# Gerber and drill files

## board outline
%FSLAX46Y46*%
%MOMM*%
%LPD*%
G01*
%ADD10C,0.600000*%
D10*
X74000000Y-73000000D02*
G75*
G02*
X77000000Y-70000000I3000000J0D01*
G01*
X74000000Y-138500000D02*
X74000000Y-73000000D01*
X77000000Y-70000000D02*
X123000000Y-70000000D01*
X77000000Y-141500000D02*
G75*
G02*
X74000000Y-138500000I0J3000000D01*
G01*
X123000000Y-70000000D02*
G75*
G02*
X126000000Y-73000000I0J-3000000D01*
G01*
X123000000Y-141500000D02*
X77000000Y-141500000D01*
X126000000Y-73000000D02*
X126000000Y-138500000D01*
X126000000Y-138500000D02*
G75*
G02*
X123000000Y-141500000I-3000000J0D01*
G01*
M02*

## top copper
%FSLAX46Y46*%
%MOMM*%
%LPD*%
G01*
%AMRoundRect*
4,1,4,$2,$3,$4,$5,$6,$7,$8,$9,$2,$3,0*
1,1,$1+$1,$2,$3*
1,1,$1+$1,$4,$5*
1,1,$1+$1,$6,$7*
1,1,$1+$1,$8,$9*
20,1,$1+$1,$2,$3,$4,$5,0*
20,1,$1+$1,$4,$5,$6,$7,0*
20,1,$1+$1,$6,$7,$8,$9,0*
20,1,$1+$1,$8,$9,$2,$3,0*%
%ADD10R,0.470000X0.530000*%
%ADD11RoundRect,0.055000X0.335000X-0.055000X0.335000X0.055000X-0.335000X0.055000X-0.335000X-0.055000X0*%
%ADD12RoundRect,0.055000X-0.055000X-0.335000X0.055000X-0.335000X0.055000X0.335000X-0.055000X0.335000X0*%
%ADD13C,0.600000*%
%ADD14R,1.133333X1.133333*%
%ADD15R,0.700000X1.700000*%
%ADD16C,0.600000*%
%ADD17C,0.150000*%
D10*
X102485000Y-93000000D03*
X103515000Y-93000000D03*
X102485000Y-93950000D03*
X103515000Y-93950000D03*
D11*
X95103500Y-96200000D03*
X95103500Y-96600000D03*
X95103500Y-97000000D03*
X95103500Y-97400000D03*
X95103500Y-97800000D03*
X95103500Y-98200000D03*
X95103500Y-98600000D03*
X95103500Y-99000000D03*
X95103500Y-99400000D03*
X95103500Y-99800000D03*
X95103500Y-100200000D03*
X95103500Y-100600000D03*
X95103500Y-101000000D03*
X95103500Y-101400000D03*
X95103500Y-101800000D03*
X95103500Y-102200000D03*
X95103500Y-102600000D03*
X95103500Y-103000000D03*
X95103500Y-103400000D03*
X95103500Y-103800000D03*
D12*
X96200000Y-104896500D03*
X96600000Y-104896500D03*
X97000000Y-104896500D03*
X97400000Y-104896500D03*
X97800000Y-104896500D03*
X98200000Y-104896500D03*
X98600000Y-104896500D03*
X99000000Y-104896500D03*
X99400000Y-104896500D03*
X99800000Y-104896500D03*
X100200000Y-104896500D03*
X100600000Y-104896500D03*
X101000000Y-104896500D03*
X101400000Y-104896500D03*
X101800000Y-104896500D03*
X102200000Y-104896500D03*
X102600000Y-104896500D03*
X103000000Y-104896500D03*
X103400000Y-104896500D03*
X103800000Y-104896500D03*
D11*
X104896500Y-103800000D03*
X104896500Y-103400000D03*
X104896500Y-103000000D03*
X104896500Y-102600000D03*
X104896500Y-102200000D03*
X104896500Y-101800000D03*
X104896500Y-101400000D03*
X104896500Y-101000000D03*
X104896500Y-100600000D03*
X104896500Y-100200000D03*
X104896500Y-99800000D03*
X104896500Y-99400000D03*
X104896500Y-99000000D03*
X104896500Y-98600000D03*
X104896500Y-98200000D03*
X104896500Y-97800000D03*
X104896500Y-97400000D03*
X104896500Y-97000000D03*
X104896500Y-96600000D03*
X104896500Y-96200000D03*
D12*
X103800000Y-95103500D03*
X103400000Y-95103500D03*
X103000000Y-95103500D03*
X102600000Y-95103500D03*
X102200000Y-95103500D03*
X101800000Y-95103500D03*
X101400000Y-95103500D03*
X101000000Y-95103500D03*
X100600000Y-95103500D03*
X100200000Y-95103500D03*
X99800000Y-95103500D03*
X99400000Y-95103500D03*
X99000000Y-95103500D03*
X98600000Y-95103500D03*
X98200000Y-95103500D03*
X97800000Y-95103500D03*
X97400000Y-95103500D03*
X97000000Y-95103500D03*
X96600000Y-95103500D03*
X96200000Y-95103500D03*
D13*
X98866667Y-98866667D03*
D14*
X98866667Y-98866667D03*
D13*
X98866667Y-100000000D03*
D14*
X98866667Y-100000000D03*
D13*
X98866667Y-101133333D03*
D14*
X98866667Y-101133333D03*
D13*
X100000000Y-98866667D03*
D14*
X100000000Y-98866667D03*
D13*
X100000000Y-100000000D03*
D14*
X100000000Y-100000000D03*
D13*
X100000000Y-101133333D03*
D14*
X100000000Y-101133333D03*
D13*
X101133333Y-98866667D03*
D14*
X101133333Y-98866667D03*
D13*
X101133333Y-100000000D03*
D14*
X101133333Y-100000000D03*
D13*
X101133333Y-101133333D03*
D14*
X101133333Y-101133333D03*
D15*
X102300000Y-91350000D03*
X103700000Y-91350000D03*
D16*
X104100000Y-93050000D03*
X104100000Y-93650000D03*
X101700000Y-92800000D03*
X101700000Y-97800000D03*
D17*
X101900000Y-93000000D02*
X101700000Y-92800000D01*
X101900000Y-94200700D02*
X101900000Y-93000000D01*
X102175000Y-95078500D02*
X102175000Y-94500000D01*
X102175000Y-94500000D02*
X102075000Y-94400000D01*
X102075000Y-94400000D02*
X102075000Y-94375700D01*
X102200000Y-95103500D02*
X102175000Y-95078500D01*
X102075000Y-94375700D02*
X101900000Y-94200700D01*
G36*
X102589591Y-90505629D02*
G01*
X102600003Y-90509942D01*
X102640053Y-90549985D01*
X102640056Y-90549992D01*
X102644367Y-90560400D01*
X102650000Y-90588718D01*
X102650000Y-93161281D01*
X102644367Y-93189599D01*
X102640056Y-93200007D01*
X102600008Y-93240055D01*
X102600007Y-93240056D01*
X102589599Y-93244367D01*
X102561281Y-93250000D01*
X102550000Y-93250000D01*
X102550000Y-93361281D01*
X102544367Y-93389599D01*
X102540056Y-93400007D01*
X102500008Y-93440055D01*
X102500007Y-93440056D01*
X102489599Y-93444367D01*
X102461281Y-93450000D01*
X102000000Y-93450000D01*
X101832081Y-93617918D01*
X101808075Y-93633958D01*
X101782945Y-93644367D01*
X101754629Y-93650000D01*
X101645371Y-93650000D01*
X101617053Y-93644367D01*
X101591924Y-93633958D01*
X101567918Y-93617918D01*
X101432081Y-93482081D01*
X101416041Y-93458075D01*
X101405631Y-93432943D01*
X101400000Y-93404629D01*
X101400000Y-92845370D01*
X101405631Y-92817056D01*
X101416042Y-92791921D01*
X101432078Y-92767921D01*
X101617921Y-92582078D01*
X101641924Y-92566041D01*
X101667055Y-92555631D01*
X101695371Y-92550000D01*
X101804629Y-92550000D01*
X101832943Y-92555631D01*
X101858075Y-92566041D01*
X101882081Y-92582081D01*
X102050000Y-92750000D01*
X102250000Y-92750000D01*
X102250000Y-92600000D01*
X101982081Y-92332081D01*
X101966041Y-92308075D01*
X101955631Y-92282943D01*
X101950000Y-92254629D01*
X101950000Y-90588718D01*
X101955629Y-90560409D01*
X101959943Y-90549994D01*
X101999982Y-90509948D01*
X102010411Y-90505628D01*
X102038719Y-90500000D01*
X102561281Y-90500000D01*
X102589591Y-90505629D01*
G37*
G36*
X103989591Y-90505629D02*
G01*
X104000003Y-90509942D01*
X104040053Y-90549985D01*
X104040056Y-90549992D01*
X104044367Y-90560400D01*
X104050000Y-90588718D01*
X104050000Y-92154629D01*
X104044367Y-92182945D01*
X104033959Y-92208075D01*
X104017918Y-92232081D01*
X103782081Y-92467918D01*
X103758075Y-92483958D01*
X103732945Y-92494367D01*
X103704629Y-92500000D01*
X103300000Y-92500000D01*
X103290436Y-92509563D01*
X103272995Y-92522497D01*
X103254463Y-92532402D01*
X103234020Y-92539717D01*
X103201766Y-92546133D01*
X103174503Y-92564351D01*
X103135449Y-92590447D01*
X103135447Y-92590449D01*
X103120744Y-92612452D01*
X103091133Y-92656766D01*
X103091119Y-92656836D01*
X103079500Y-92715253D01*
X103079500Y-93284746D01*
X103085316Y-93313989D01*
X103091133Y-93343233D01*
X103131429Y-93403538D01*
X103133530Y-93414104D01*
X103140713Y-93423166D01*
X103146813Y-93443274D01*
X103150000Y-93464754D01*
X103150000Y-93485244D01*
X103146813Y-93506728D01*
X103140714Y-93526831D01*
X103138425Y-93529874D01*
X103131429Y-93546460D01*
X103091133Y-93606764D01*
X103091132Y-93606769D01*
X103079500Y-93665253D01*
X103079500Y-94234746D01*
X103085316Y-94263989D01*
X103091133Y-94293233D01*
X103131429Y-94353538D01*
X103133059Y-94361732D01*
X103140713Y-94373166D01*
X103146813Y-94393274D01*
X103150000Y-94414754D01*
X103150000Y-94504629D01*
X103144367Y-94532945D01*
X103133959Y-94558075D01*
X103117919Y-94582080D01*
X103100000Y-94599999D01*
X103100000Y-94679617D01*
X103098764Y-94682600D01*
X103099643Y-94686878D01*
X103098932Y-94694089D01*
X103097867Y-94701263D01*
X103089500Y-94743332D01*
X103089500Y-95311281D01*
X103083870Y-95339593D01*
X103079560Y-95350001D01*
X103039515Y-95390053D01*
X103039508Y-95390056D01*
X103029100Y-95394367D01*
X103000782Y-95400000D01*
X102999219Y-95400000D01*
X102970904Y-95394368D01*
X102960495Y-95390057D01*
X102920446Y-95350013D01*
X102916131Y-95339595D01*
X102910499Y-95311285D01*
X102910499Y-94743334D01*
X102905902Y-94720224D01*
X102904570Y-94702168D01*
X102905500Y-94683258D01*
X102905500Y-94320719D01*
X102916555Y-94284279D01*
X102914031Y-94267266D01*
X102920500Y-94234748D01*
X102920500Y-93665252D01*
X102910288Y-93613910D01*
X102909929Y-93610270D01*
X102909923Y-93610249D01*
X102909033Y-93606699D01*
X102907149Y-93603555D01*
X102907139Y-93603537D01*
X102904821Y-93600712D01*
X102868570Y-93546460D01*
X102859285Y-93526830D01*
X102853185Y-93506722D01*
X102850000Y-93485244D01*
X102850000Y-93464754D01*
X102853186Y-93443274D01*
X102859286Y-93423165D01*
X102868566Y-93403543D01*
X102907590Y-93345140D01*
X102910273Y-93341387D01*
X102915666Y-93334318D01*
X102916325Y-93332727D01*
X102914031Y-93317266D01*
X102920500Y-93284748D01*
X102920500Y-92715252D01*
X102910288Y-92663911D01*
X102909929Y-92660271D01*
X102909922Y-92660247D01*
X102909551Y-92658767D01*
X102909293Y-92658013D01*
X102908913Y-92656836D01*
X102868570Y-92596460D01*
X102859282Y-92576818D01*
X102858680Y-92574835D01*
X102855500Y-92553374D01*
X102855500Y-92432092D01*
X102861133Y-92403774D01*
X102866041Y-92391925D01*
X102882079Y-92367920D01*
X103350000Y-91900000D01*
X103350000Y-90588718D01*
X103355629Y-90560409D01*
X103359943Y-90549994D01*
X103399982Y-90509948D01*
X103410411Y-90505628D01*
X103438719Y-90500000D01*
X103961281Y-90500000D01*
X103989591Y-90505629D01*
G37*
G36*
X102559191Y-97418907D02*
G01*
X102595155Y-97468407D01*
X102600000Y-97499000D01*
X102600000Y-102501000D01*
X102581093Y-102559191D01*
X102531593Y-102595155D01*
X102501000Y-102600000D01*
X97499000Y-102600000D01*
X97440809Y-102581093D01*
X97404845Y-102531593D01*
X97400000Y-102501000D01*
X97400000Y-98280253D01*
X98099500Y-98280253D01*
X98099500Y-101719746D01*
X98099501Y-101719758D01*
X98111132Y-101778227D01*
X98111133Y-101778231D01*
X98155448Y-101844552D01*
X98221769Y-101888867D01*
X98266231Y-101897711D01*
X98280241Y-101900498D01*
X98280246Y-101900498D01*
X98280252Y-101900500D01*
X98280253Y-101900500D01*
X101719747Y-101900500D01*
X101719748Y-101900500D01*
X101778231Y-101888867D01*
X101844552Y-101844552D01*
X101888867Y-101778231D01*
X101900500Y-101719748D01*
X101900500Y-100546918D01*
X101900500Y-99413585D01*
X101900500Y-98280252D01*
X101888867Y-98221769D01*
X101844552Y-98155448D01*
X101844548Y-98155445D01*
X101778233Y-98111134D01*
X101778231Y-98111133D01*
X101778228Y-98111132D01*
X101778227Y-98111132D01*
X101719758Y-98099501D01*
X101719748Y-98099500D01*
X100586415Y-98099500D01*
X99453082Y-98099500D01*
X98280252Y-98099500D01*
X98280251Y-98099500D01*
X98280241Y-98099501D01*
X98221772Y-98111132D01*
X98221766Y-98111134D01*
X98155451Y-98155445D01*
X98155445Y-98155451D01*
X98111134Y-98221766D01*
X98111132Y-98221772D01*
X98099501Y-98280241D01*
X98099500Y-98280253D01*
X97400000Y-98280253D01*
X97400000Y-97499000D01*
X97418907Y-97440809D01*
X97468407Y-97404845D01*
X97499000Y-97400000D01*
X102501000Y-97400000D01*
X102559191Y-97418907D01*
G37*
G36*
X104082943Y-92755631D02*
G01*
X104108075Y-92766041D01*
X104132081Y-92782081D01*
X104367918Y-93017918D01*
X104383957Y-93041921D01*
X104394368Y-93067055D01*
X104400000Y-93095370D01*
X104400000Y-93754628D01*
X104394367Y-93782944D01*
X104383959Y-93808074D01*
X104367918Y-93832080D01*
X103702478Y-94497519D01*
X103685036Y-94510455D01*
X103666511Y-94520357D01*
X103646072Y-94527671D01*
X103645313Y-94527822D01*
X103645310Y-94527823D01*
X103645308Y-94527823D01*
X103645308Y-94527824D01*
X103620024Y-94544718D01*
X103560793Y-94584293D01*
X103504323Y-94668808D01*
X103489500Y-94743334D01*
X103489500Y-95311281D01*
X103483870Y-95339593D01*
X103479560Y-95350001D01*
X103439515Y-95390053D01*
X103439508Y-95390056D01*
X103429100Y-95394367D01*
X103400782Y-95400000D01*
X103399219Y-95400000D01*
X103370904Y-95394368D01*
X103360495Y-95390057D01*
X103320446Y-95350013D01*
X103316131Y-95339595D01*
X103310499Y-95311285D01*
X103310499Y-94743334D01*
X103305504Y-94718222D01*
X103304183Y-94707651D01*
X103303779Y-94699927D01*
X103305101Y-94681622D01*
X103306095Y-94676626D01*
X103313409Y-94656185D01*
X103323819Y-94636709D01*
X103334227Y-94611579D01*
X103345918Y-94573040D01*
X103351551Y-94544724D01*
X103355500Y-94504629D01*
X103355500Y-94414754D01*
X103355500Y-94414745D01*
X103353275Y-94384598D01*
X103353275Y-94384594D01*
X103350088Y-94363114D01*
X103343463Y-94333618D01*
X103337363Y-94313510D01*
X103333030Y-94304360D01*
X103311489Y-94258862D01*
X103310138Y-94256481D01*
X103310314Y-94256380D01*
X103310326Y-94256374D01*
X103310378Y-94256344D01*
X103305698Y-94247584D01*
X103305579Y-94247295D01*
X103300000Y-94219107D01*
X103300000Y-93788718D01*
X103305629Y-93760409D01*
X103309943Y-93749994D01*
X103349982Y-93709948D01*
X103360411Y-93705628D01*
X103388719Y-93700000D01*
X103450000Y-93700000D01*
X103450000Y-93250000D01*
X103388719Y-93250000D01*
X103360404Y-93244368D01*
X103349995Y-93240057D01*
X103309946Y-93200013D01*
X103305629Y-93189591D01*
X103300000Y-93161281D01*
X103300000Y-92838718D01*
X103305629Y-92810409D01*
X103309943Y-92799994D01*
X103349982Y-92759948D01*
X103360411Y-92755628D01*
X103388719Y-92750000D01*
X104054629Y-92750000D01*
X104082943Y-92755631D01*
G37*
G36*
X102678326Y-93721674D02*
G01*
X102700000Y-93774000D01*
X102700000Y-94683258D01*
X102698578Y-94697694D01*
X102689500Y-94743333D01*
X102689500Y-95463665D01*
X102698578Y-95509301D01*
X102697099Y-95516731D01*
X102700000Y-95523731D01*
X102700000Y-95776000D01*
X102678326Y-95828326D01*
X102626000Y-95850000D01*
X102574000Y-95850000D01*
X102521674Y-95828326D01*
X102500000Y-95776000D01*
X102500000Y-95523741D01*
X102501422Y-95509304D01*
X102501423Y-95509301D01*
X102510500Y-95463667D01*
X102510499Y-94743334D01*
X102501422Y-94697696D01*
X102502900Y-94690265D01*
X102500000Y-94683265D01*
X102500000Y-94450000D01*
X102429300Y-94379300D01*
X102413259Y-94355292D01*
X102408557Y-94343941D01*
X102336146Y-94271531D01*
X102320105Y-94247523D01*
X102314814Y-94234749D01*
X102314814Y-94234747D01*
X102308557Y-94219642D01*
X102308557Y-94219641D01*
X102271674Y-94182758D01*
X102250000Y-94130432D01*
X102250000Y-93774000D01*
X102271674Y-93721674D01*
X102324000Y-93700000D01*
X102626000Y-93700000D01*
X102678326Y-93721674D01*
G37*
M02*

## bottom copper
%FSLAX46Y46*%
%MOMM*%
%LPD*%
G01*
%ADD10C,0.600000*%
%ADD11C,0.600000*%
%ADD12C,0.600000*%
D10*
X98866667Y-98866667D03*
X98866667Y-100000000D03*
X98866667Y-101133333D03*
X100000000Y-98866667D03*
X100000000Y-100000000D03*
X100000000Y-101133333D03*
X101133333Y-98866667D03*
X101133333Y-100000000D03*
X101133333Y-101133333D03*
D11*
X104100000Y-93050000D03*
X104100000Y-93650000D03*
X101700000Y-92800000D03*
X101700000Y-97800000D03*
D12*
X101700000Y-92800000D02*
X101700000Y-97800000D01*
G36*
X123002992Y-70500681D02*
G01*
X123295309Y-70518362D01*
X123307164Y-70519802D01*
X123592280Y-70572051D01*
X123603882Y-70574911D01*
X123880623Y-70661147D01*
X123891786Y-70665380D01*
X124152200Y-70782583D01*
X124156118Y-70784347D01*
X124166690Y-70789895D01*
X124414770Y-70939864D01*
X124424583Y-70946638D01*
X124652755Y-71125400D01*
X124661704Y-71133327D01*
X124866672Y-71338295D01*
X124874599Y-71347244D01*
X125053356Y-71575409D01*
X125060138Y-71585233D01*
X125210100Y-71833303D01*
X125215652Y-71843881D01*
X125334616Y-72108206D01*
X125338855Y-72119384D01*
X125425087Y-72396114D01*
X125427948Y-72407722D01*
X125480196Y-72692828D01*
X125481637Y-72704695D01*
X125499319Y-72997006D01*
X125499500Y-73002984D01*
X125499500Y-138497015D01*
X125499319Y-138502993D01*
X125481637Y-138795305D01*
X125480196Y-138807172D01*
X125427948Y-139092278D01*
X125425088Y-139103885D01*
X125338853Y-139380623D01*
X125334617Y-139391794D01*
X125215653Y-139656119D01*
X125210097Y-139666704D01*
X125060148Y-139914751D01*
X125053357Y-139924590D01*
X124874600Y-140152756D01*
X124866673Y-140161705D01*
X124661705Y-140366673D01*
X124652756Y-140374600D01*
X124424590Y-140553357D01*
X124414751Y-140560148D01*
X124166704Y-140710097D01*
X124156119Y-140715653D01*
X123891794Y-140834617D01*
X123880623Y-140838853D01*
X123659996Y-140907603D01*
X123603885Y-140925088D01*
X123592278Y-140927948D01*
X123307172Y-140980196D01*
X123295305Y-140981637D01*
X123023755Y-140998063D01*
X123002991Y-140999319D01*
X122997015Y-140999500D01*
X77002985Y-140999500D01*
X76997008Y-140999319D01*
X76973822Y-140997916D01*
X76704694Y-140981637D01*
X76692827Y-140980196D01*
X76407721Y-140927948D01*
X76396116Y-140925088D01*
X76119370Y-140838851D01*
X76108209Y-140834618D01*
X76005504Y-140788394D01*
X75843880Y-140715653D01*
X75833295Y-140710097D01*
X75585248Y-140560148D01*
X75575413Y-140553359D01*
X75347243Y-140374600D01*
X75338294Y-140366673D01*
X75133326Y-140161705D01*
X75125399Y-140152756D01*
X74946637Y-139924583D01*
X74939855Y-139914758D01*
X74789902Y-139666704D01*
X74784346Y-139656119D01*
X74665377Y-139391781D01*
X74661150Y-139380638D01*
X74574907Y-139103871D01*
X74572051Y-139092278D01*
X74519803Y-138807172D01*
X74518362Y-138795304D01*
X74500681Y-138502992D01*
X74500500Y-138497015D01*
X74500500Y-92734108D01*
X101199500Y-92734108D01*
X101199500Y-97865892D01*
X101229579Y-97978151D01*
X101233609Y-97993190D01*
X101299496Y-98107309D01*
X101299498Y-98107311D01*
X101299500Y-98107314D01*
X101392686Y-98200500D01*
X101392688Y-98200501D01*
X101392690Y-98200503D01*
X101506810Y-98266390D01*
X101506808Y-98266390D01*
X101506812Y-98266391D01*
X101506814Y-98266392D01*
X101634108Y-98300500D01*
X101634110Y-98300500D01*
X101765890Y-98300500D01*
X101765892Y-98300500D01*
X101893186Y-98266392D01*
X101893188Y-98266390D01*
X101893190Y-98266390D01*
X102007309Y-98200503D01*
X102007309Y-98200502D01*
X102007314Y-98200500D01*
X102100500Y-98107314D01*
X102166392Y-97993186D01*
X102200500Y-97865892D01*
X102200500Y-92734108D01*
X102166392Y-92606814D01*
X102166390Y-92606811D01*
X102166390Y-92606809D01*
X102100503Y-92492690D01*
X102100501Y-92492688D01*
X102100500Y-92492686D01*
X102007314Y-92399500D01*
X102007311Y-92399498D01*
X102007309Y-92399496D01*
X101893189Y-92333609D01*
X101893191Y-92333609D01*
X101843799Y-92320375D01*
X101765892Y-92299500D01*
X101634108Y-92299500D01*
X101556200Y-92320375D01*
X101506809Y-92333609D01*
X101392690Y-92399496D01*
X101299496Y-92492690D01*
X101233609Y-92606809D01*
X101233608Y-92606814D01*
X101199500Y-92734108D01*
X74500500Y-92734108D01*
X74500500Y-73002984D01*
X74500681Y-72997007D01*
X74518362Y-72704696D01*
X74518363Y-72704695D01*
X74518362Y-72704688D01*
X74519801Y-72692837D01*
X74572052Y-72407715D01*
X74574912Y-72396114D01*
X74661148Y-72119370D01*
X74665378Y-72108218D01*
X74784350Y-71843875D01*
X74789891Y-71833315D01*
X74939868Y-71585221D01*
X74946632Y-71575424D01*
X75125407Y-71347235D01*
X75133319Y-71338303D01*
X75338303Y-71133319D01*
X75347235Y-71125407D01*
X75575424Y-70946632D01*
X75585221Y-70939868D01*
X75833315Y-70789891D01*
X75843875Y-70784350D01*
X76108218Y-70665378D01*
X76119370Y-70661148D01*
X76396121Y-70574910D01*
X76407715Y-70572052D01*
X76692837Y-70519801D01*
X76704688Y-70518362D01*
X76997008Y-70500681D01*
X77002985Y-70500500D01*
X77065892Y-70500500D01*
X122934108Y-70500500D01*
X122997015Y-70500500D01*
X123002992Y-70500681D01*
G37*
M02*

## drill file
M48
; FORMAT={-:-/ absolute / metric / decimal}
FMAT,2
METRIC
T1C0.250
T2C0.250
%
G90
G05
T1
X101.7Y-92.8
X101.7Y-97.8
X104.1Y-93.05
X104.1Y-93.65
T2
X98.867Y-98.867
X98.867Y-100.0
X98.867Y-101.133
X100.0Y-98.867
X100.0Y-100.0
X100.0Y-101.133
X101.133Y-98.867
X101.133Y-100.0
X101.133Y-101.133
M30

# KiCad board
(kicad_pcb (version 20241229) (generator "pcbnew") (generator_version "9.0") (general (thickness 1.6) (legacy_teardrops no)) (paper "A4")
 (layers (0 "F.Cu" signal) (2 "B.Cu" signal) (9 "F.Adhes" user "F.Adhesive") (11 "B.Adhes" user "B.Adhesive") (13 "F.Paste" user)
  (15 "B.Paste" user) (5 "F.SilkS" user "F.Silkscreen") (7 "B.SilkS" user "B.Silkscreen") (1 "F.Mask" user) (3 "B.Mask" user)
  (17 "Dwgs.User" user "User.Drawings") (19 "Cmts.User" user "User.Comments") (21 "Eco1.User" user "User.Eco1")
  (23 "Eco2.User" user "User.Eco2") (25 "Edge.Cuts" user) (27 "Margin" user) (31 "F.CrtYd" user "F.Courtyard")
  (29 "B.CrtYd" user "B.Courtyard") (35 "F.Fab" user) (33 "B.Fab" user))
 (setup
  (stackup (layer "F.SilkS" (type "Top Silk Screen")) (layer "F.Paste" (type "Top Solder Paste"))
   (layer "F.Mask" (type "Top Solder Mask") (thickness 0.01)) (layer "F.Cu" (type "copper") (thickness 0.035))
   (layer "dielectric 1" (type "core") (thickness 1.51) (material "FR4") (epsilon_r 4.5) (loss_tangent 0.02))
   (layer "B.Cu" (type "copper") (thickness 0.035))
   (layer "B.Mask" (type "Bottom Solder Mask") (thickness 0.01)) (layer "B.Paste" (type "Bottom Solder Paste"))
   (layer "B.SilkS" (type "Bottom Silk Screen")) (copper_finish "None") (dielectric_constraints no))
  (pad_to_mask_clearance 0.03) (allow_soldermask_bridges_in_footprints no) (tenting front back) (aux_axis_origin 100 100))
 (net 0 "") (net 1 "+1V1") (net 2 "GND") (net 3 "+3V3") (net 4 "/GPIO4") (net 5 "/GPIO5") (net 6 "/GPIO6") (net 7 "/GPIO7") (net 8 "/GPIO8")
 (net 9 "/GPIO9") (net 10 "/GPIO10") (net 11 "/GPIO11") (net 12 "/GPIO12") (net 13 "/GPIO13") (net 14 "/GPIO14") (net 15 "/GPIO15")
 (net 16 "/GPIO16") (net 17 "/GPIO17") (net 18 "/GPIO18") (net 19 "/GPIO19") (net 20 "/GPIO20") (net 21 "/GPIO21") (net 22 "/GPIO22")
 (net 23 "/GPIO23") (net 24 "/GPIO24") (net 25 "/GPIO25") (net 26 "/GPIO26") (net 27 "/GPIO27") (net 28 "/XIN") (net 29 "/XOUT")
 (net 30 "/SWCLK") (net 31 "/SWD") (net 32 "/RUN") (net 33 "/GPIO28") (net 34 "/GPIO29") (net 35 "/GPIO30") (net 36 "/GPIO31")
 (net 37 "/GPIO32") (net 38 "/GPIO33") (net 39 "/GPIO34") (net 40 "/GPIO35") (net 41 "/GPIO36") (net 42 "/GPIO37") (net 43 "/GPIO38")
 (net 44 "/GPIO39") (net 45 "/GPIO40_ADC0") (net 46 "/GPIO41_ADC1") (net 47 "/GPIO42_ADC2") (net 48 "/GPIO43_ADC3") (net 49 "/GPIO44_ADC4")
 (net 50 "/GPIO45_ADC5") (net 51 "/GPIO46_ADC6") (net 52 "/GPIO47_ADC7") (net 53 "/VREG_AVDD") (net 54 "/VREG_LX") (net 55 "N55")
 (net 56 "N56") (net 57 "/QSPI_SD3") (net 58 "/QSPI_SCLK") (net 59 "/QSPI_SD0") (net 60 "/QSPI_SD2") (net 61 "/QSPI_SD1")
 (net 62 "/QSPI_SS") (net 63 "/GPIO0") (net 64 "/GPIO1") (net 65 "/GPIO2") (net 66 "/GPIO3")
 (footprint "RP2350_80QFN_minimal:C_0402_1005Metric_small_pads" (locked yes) (layer "F.Cu") (at 103 93)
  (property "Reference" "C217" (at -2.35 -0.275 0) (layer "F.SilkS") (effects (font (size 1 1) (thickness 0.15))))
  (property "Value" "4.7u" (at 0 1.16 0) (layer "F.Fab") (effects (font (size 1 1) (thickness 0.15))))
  (pad "1" smd rect (at -0.515 0) (size 0.47 0.53) (layers "F.Cu" "F.Mask" "F.Paste") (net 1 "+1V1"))
  (pad "2" smd rect (at 0.515 0) (size 0.47 0.53) (layers "F.Cu" "F.Mask" "F.Paste") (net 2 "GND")))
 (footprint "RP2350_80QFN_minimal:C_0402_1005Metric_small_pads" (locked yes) (layer "F.Cu") (at 103 93.95)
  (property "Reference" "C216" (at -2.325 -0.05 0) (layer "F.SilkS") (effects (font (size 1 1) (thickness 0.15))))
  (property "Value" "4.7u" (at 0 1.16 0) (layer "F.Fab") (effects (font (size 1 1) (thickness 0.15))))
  (pad "1" smd rect (at -0.515 0) (size 0.47 0.53) (layers "F.Cu" "F.Mask" "F.Paste") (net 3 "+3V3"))
  (pad "2" smd rect (at 0.515 0) (size 0.47 0.53) (layers "F.Cu" "F.Mask" "F.Paste") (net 2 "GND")))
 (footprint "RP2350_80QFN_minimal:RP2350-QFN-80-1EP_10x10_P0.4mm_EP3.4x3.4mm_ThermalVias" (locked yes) (layer "F.Cu") (at 100 100)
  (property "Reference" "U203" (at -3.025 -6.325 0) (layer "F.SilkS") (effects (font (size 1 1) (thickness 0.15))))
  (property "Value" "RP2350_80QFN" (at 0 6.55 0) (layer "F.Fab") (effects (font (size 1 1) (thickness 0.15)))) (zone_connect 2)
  (pad "" smd roundrect (at -0.7 -0.7) (size 1.2 1.2) (layers "F.Paste") (roundrect_rratio 0.2083333333) (zone_connect 2))
  (pad "" smd roundrect (at -0.7 0.7) (size 1.2 1.2) (layers "F.Paste") (roundrect_rratio 0.2083333333) (zone_connect 2))
  (pad "" smd roundrect (at 0.7 -0.7) (size 1.2 1.2) (layers "F.Paste") (roundrect_rratio 0.2083333333) (zone_connect 2))
  (pad "" smd roundrect (at 0.7 0.7) (size 1.2 1.2) (layers "F.Paste") (roundrect_rratio 0.2083333333) (zone_connect 2))
  (pad "1" smd roundrect (at -4.8965 -3.8 90) (size 0.22 0.78) (layers "F.Cu" "F.Mask" "F.Paste") (roundrect_rratio 0.25) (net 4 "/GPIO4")
   (thermal_bridge_angle 45))
  (pad "2" smd roundrect (at -4.8965 -3.4 90) (size 0.22 0.78) (layers "F.Cu" "F.Mask" "F.Paste") (roundrect_rratio 0.25) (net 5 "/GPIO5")
   (thermal_bridge_angle 45))
  (pad "3" smd roundrect (at -4.8965 -3 90) (size 0.22 0.78) (layers "F.Cu" "F.Mask" "F.Paste") (roundrect_rratio 0.25) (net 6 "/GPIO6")
   (thermal_bridge_angle 45))
  (pad "4" smd roundrect (at -4.8965 -2.6 90) (size 0.22 0.78) (layers "F.Cu" "F.Mask" "F.Paste") (roundrect_rratio 0.25) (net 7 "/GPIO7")
   (thermal_bridge_angle 45))
  (pad "5" smd roundrect (at -4.8965 -2.2 90) (size 0.22 0.78) (layers "F.Cu" "F.Mask" "F.Paste") (roundrect_rratio 0.25) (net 3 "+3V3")
   (thermal_bridge_angle 45))
  (pad "6" smd roundrect (at -4.8965 -1.8 90) (size 0.22 0.78) (layers "F.Cu" "F.Mask" "F.Paste") (roundrect_rratio 0.25) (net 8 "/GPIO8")
   (thermal_bridge_angle 45))
  (pad "7" smd roundrect (at -4.8965 -1.4 90) (size 0.22 0.78) (layers "F.Cu" "F.Mask" "F.Paste") (roundrect_rratio 0.25) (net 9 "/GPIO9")
   (thermal_bridge_angle 45))
  (pad "8" smd roundrect (at -4.8965 -1 90) (size 0.22 0.78) (layers "F.Cu" "F.Mask" "F.Paste") (roundrect_rratio 0.25) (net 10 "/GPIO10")
   (thermal_bridge_angle 45))
  (pad "9" smd roundrect (at -4.8965 -0.6 90) (size 0.22 0.78) (layers "F.Cu" "F.Mask" "F.Paste") (roundrect_rratio 0.25) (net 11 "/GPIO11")
   (thermal_bridge_angle 45))
  (pad "10" smd roundrect (at -4.8965 -0.2 90) (size 0.22 0.78) (layers "F.Cu" "F.Mask" "F.Paste") (roundrect_rratio 0.25) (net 1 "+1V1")
   (thermal_bridge_angle 45))
  (pad "11" smd roundrect (at -4.8965 0.2 90) (size 0.22 0.78) (layers "F.Cu" "F.Mask" "F.Paste") (roundrect_rratio 0.25) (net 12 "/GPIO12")
   (thermal_bridge_angle 45))
  (pad "12" smd roundrect (at -4.8965 0.6 90) (size 0.22 0.78) (layers "F.Cu" "F.Mask" "F.Paste") (roundrect_rratio 0.25) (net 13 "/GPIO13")
   (thermal_bridge_angle 45))
  (pad "13" smd roundrect (at -4.8965 1 90) (size 0.22 0.78) (layers "F.Cu" "F.Mask" "F.Paste") (roundrect_rratio 0.25) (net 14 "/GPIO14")
   (thermal_bridge_angle 45))
  (pad "14" smd roundrect (at -4.8965 1.4 90) (size 0.22 0.78) (layers "F.Cu" "F.Mask" "F.Paste") (roundrect_rratio 0.25) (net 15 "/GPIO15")
   (thermal_bridge_angle 45))
  (pad "15" smd roundrect (at -4.8965 1.8 90) (size 0.22 0.78) (layers "F.Cu" "F.Mask" "F.Paste") (roundrect_rratio 0.25) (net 3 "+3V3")
   (thermal_bridge_angle 45))
  (pad "16" smd roundrect (at -4.8965 2.2 90) (size 0.22 0.78) (layers "F.Cu" "F.Mask" "F.Paste") (roundrect_rratio 0.25) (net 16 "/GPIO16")
   (thermal_bridge_angle 45))
  (pad "17" smd roundrect (at -4.8965 2.6 90) (size 0.22 0.78) (layers "F.Cu" "F.Mask" "F.Paste") (roundrect_rratio 0.25) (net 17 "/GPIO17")
   (thermal_bridge_angle 45))
  (pad "18" smd roundrect (at -4.8965 3 90) (size 0.22 0.78) (layers "F.Cu" "F.Mask" "F.Paste") (roundrect_rratio 0.25) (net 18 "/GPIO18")
   (thermal_bridge_angle 45))
  (pad "19" smd roundrect (at -4.8965 3.4 90) (size 0.22 0.78) (layers "F.Cu" "F.Mask" "F.Paste") (roundrect_rratio 0.25) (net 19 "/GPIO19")
   (thermal_bridge_angle 45))
  (pad "20" smd roundrect (at -4.8965 3.8 90) (size 0.22 0.78) (layers "F.Cu" "F.Mask" "F.Paste") (roundrect_rratio 0.25) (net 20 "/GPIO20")
   (thermal_bridge_angle 45))
  (pad "21" smd roundrect (at -3.8 4.8965) (size 0.22 0.78) (layers "F.Cu" "F.Mask" "F.Paste") (roundrect_rratio 0.25) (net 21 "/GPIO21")
   (thermal_bridge_angle 45))
  (pad "22" smd roundrect (at -3.4 4.8965) (size 0.22 0.78) (layers "F.Cu" "F.Mask" "F.Paste") (roundrect_rratio 0.25) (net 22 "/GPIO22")
   (thermal_bridge_angle 45))
  (pad "23" smd roundrect (at -3 4.8965) (size 0.22 0.78) (layers "F.Cu" "F.Mask" "F.Paste") (roundrect_rratio 0.25) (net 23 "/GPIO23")
   (thermal_bridge_angle 45))
  (pad "24" smd roundrect (at -2.6 4.8965) (size 0.22 0.78) (layers "F.Cu" "F.Mask" "F.Paste") (roundrect_rratio 0.25) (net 3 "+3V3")
   (thermal_bridge_angle 45))
  (pad "25" smd roundrect (at -2.2 4.8965) (size 0.22 0.78) (layers "F.Cu" "F.Mask" "F.Paste") (roundrect_rratio 0.25) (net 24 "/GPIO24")
   (thermal_bridge_angle 45))
  (pad "26" smd roundrect (at -1.8 4.8965) (size 0.22 0.78) (layers "F.Cu" "F.Mask" "F.Paste") (roundrect_rratio 0.25) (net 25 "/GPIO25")
   (thermal_bridge_angle 45))
  (pad "27" smd roundrect (at -1.4 4.8965) (size 0.22 0.78) (layers "F.Cu" "F.Mask" "F.Paste") (roundrect_rratio 0.25) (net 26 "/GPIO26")
   (thermal_bridge_angle 45))
  (pad "28" smd roundrect (at -1 4.8965) (size 0.22 0.78) (layers "F.Cu" "F.Mask" "F.Paste") (roundrect_rratio 0.25) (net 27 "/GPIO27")
   (thermal_bridge_angle 45))
  (pad "29" smd roundrect (at -0.6 4.8965) (size 0.22 0.78) (layers "F.Cu" "F.Mask" "F.Paste") (roundrect_rratio 0.25) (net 3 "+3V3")
   (thermal_bridge_angle 45))
  (pad "30" smd roundrect (at -0.2 4.8965) (size 0.22 0.78) (layers "F.Cu" "F.Mask" "F.Paste") (roundrect_rratio 0.25) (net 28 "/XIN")
   (thermal_bridge_angle 45))
  (pad "31" smd roundrect (at 0.2 4.8965) (size 0.22 0.78) (layers "F.Cu" "F.Mask" "F.Paste") (roundrect_rratio 0.25) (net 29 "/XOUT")
   (thermal_bridge_angle 45))
  (pad "32" smd roundrect (at 0.6 4.8965) (size 0.22 0.78) (layers "F.Cu" "F.Mask" "F.Paste") (roundrect_rratio 0.25) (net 1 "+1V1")
   (thermal_bridge_angle 45))
  (pad "33" smd roundrect (at 1 4.8965) (size 0.22 0.78) (layers "F.Cu" "F.Mask" "F.Paste") (roundrect_rratio 0.25) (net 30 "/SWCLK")
   (thermal_bridge_angle 45))
  (pad "34" smd roundrect (at 1.4 4.8965) (size 0.22 0.78) (layers "F.Cu" "F.Mask" "F.Paste") (roundrect_rratio 0.25) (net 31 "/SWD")
   (thermal_bridge_angle 45))
  (pad "35" smd roundrect (at 1.8 4.8965) (size 0.22 0.78) (layers "F.Cu" "F.Mask" "F.Paste") (roundrect_rratio 0.25) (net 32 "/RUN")
   (thermal_bridge_angle 45))
  (pad "36" smd roundrect (at 2.2 4.8965) (size 0.22 0.78) (layers "F.Cu" "F.Mask" "F.Paste") (roundrect_rratio 0.25) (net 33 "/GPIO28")
   (thermal_bridge_angle 45))
  (pad "37" smd roundrect (at 2.6 4.8965) (size 0.22 0.78) (layers "F.Cu" "F.Mask" "F.Paste") (roundrect_rratio 0.25) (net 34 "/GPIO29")
   (thermal_bridge_angle 45))
  (pad "38" smd roundrect (at 3 4.8965) (size 0.22 0.78) (layers "F.Cu" "F.Mask" "F.Paste") (roundrect_rratio 0.25) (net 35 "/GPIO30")
   (thermal_bridge_angle 45))
  (pad "39" smd roundrect (at 3.4 4.8965) (size 0.22 0.78) (layers "F.Cu" "F.Mask" "F.Paste") (roundrect_rratio 0.25) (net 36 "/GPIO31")
   (thermal_bridge_angle 45))
  (pad "40" smd roundrect (at 3.8 4.8965) (size 0.22 0.78) (layers "F.Cu" "F.Mask" "F.Paste") (roundrect_rratio 0.25) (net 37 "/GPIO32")
   (thermal_bridge_angle 45))
  (pad "41" smd roundrect (at 4.8965 3.8 90) (size 0.22 0.78) (layers "F.Cu" "F.Mask" "F.Paste") (roundrect_rratio 0.25) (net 3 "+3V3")
   (thermal_bridge_angle 45))
  (pad "42" smd roundrect (at 4.8965 3.4 90) (size 0.22 0.78) (layers "F.Cu" "F.Mask" "F.Paste") (roundrect_rratio 0.25) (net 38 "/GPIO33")
   (thermal_bridge_angle 45))
  (pad "43" smd roundrect (at 4.8965 3 90) (size 0.22 0.78) (layers "F.Cu" "F.Mask" "F.Paste") (roundrect_rratio 0.25) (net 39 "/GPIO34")
   (thermal_bridge_angle 45))
  (pad "44" smd roundrect (at 4.8965 2.6 90) (size 0.22 0.78) (layers "F.Cu" "F.Mask" "F.Paste") (roundrect_rratio 0.25) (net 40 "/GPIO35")
   (thermal_bridge_angle 45))
  (pad "45" smd roundrect (at 4.8965 2.2 90) (size 0.22 0.78) (layers "F.Cu" "F.Mask" "F.Paste") (roundrect_rratio 0.25) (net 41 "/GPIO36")
   (thermal_bridge_angle 45))
  (pad "46" smd roundrect (at 4.8965 1.8 90) (size 0.22 0.78) (layers "F.Cu" "F.Mask" "F.Paste") (roundrect_rratio 0.25) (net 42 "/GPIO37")
   (thermal_bridge_angle 45))
  (pad "47" smd roundrect (at 4.8965 1.4 90) (size 0.22 0.78) (layers "F.Cu" "F.Mask" "F.Paste") (roundrect_rratio 0.25) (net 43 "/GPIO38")
   (thermal_bridge_angle 45))
  (pad "48" smd roundrect (at 4.8965 1 90) (size 0.22 0.78) (layers "F.Cu" "F.Mask" "F.Paste") (roundrect_rratio 0.25) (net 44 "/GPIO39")
   (thermal_bridge_angle 45))
  (pad "49" smd roundrect (at 4.8965 0.6 90) (size 0.22 0.78) (layers "F.Cu" "F.Mask" "F.Paste") (roundrect_rratio 0.25)
   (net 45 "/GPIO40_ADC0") (thermal_bridge_angle 45))
  (pad "50" smd roundrect (at 4.8965 0.2 90) (size 0.22 0.78) (layers "F.Cu" "F.Mask" "F.Paste") (roundrect_rratio 0.25) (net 3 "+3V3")
   (thermal_bridge_angle 45))
  (pad "51" smd roundrect (at 4.8965 -0.2 90) (size 0.22 0.78) (layers "F.Cu" "F.Mask" "F.Paste") (roundrect_rratio 0.25) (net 1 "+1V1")
   (thermal_bridge_angle 45))
  (pad "52" smd roundrect (at 4.8965 -0.6 90) (size 0.22 0.78) (layers "F.Cu" "F.Mask" "F.Paste") (roundrect_rratio 0.25)
   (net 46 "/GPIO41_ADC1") (thermal_bridge_angle 45))
  (pad "53" smd roundrect (at 4.8965 -1 90) (size 0.22 0.78) (layers "F.Cu" "F.Mask" "F.Paste") (roundrect_rratio 0.25)
   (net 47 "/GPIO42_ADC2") (thermal_bridge_angle 45))
  (pad "54" smd roundrect (at 4.8965 -1.4 90) (size 0.22 0.78) (layers "F.Cu" "F.Mask" "F.Paste") (roundrect_rratio 0.25)
   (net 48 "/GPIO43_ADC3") (thermal_bridge_angle 45))
  (pad "55" smd roundrect (at 4.8965 -1.8 90) (size 0.22 0.78) (layers "F.Cu" "F.Mask" "F.Paste") (roundrect_rratio 0.25)
   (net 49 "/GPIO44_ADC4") (thermal_bridge_angle 45))
  (pad "56" smd roundrect (at 4.8965 -2.2 90) (size 0.22 0.78) (layers "F.Cu" "F.Mask" "F.Paste") (roundrect_rratio 0.25)
   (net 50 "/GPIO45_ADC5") (thermal_bridge_angle 45))
  (pad "57" smd roundrect (at 4.8965 -2.6 90) (size 0.22 0.78) (layers "F.Cu" "F.Mask" "F.Paste") (roundrect_rratio 0.25)
   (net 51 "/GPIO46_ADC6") (thermal_bridge_angle 45))
  (pad "58" smd roundrect (at 4.8965 -3 90) (size 0.22 0.78) (layers "F.Cu" "F.Mask" "F.Paste") (roundrect_rratio 0.25)
   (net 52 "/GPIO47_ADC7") (thermal_bridge_angle 45))
  (pad "59" smd roundrect (at 4.8965 -3.4 90) (size 0.22 0.78) (layers "F.Cu" "F.Mask" "F.Paste") (roundrect_rratio 0.25) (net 3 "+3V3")
   (thermal_bridge_angle 45))
  (pad "60" smd roundrect (at 4.8965 -3.8 90) (size 0.22 0.78) (layers "F.Cu" "F.Mask" "F.Paste") (roundrect_rratio 0.25) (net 3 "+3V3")
   (thermal_bridge_angle 45))
  (pad "61" smd roundrect (at 3.8 -4.8965) (size 0.22 0.78) (layers "F.Cu" "F.Mask" "F.Paste") (roundrect_rratio 0.25) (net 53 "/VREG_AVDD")
   (thermal_bridge_angle 45))
  (pad "62" smd roundrect (at 3.4 -4.8965) (size 0.22 0.78) (layers "F.Cu" "F.Mask" "F.Paste") (roundrect_rratio 0.25) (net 2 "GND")
   (thermal_bridge_angle 45))
  (pad "63" smd roundrect (at 3 -4.8965) (size 0.22 0.78) (layers "F.Cu" "F.Mask" "F.Paste") (roundrect_rratio 0.25) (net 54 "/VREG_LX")
   (thermal_bridge_angle 45))
  (pad "64" smd roundrect (at 2.6 -4.8965) (size 0.22 0.78) (layers "F.Cu" "F.Mask" "F.Paste") (roundrect_rratio 0.25) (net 3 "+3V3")
   (thermal_bridge_angle 45))
  (pad "65" smd roundrect (at 2.2 -4.8965) (size 0.22 0.78) (layers "F.Cu" "F.Mask" "F.Paste") (roundrect_rratio 0.25) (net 1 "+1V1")
   (thermal_bridge_angle 45))
  (pad "66" smd roundrect (at 1.8 -4.8965) (size 0.22 0.78) (layers "F.Cu" "F.Mask" "F.Paste") (roundrect_rratio 0.25) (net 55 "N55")
   (thermal_bridge_angle 45))
  (pad "67" smd roundrect (at 1.4 -4.8965) (size 0.22 0.78) (layers "F.Cu" "F.Mask" "F.Paste") (roundrect_rratio 0.25) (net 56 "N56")
   (thermal_bridge_angle 45))
  (pad "68" smd roundrect (at 1 -4.8965) (size 0.22 0.78) (layers "F.Cu" "F.Mask" "F.Paste") (roundrect_rratio 0.25) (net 3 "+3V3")
   (thermal_bridge_angle 45))
  (pad "69" smd roundrect (at 0.6 -4.8965) (size 0.22 0.78) (layers "F.Cu" "F.Mask" "F.Paste") (roundrect_rratio 0.25) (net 3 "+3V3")
   (thermal_bridge_angle 45))
  (pad "70" smd roundrect (at 0.2 -4.8965) (size 0.22 0.78) (layers "F.Cu" "F.Mask" "F.Paste") (roundrect_rratio 0.25) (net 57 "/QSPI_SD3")
   (thermal_bridge_angle 45))
  (pad "71" smd roundrect (at -0.2 -4.8965) (size 0.22 0.78) (layers "F.Cu" "F.Mask" "F.Paste") (roundrect_rratio 0.25)
   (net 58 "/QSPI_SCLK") (thermal_bridge_angle 45))
  (pad "72" smd roundrect (at -0.6 -4.8965) (size 0.22 0.78) (layers "F.Cu" "F.Mask" "F.Paste") (roundrect_rratio 0.25) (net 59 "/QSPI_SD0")
   (thermal_bridge_angle 45))
  (pad "73" smd roundrect (at -1 -4.8965) (size 0.22 0.78) (layers "F.Cu" "F.Mask" "F.Paste") (roundrect_rratio 0.25) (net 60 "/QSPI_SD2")
   (thermal_bridge_angle 45))
  (pad "74" smd roundrect (at -1.4 -4.8965) (size 0.22 0.78) (layers "F.Cu" "F.Mask" "F.Paste") (roundrect_rratio 0.25) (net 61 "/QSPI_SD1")
   (thermal_bridge_angle 45))
  (pad "75" smd roundrect (at -1.8 -4.8965) (size 0.22 0.78) (layers "F.Cu" "F.Mask" "F.Paste") (roundrect_rratio 0.25) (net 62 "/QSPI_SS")
   (thermal_bridge_angle 45))
  (pad "76" smd roundrect (at -2.2 -4.8965) (size 0.22 0.78) (layers "F.Cu" "F.Mask" "F.Paste") (roundrect_rratio 0.25) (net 3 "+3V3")
   (thermal_bridge_angle 45))
  (pad "77" smd roundrect (at -2.6 -4.8965) (size 0.22 0.78) (layers "F.Cu" "F.Mask" "F.Paste") (roundrect_rratio 0.25) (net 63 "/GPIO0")
   (thermal_bridge_angle 45))
  (pad "78" smd roundrect (at -3 -4.8965) (size 0.22 0.78) (layers "F.Cu" "F.Mask" "F.Paste") (roundrect_rratio 0.25) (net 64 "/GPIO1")
   (thermal_bridge_angle 45))
  (pad "79" smd roundrect (at -3.4 -4.8965) (size 0.22 0.78) (layers "F.Cu" "F.Mask" "F.Paste") (roundrect_rratio 0.25) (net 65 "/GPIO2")
   (thermal_bridge_angle 45))
  (pad "80" smd roundrect (at -3.8 -4.8965) (size 0.22 0.78) (layers "F.Cu" "F.Mask" "F.Paste") (roundrect_rratio 0.25) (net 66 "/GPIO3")
   (thermal_bridge_angle 45))
  (pad "81" thru_hole circle (at -1.133333 -1.133333) (size 0.6 0.6) (drill 0.25) (layers "*.Cu" "*.Mask") (remove_unused_layers no)
   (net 2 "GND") (zone_connect 2))
  (pad "81" smd rect (at -1.133333 -1.133333) (size 1.133333 1.133333) (layers "F.Cu" "F.Mask" "F.Paste") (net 2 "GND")
   (solder_paste_margin -0.5) (thermal_bridge_angle 45))
  (pad "81" thru_hole circle (at -1.133333 0) (size 0.6 0.6) (drill 0.25) (layers "*.Cu" "*.Mask") (remove_unused_layers no) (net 2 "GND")
   (zone_connect 2))
  (pad "81" smd rect (at -1.133333 0) (size 1.133333 1.133333) (layers "F.Cu" "F.Mask" "F.Paste") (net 2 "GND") (solder_paste_margin -0.5)
   (thermal_bridge_angle 45))
  (pad "81" thru_hole circle (at -1.133333 1.133333) (size 0.6 0.6) (drill 0.25) (layers "*.Cu" "*.Mask") (remove_unused_layers no)
   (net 2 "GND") (zone_connect 2))
  (pad "81" smd rect (at -1.133333 1.133333) (size 1.133333 1.133333) (layers "F.Cu" "F.Mask" "F.Paste") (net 2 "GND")
   (solder_paste_margin -0.5) (thermal_bridge_angle 45))
  (pad "81" thru_hole circle (at 0 -1.133333) (size 0.6 0.6) (drill 0.25) (layers "*.Cu" "*.Mask") (remove_unused_layers no) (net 2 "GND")
   (zone_connect 2))
  (pad "81" smd rect (at 0 -1.133333) (size 1.133333 1.133333) (layers "F.Cu" "F.Mask" "F.Paste") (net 2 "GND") (solder_paste_margin -0.5)
   (thermal_bridge_angle 45))
  (pad "81" thru_hole circle (at 0 0) (size 0.6 0.6) (drill 0.25) (layers "*.Cu" "*.Mask") (remove_unused_layers no) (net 2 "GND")
   (zone_connect 2))
  (pad "81" smd rect (at 0 0) (size 1.133333 1.133333) (layers "F.Cu" "F.Mask" "F.Paste") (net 2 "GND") (solder_paste_margin -0.5)
   (thermal_bridge_angle 45))
  (pad "81" thru_hole circle (at 0 1.133333) (size 0.6 0.6) (drill 0.25) (layers "*.Cu" "*.Mask") (remove_unused_layers no) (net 2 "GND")
   (zone_connect 2))
  (pad "81" smd rect (at 0 1.133333) (size 1.133333 1.133333) (layers "F.Cu" "F.Mask" "F.Paste") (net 2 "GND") (solder_paste_margin -0.5)
   (thermal_bridge_angle 45))
  (pad "81" thru_hole circle (at 1.133333 -1.133333) (size 0.6 0.6) (drill 0.25) (layers "*.Cu" "*.Mask") (remove_unused_layers no)
   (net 2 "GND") (zone_connect 2))
  (pad "81" smd rect (at 1.133333 -1.133333) (size 1.133333 1.133333) (layers "F.Cu" "F.Mask" "F.Paste") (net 2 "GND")
   (solder_paste_margin -0.5) (thermal_bridge_angle 45))
  (pad "81" thru_hole circle (at 1.133333 0) (size 0.6 0.6) (drill 0.25) (layers "*.Cu" "*.Mask") (remove_unused_layers no) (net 2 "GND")
   (zone_connect 2))
  (pad "81" smd rect (at 1.133333 0) (size 1.133333 1.133333) (layers "F.Cu" "F.Mask" "F.Paste") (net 2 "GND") (solder_paste_margin -0.5)
   (thermal_bridge_angle 45))
  (pad "81" thru_hole circle (at 1.133333 1.133333) (size 0.6 0.6) (drill 0.25) (layers "*.Cu" "*.Mask") (remove_unused_layers no)
   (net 2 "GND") (zone_connect 2))
  (pad "81" smd rect (at 1.133333 1.133333) (size 1.133333 1.133333) (layers "F.Cu" "F.Mask" "F.Paste") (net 2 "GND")
   (solder_paste_margin -0.5) (thermal_bridge_angle 45)))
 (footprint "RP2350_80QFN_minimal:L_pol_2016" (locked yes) (layer "F.Cu") (at 103 91.35)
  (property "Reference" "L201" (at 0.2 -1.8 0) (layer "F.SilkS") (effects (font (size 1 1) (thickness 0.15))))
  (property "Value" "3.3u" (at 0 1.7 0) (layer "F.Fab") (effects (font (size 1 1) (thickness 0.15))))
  (pad "1" smd rect (at -0.7 0) (size 0.7 1.7) (layers "F.Cu" "F.Mask" "F.Paste") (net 1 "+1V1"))
  (pad "2" smd rect (at 0.7 0) (size 0.7 1.7) (layers "F.Cu" "F.Mask" "F.Paste") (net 54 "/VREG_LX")))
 (gr_arc (start 74 73) (mid 74.87868 70.87868) (end 77 70) (stroke (width 0.6) (type solid)) (layer "Edge.Cuts"))
 (gr_line (start 74 138.5) (end 74 73) (stroke (width 0.6) (type solid)) (layer "Edge.Cuts"))
 (gr_line (start 77 70) (end 123 70) (stroke (width 0.6) (type solid)) (layer "Edge.Cuts"))
 (gr_arc (start 77 141.5) (mid 74.878679 140.621321) (end 74 138.5) (stroke (width 0.6) (type solid)) (layer "Edge.Cuts"))
 (gr_arc (start 123 70) (mid 125.12132 70.87868) (end 126 73) (stroke (width 0.6) (type solid)) (layer "Edge.Cuts"))
 (gr_line (start 123 141.5) (end 77 141.5) (stroke (width 0.6) (type solid)) (layer "Edge.Cuts"))
 (gr_line (start 126 73) (end 126 138.5) (stroke (width 0.6) (type solid)) (layer "Edge.Cuts"))
 (gr_arc (start 126 138.5) (mid 125.121321 140.621321) (end 123 141.5) (stroke (width 0.6) (type solid)) (layer "Edge.Cuts"))
 (via (at 104.1 93.05) (size 0.6) (drill 0.25) (layers "F.Cu" "B.Cu") (locked yes) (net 2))
 (via (at 104.1 93.65) (size 0.6) (drill 0.25) (layers "F.Cu" "B.Cu") (locked yes) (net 2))
 (segment (start 101.9 93) (end 101.7 92.8) (width 0.15) (locked yes) (layer "F.Cu") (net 1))
 (segment (start 101.9 94.2007) (end 101.9 93) (width 0.15) (locked yes) (layer "F.Cu") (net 1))
 (segment (start 102.175 95.0785) (end 102.175 94.5) (width 0.15) (locked yes) (layer "F.Cu") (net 1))
 (segment (start 102.175 94.5) (end 102.075 94.4) (width 0.15) (locked yes) (layer "F.Cu") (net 1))
 (segment (start 102.075 94.4) (end 102.075 94.3757) (width 0.15) (locked yes) (layer "F.Cu") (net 1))
 (segment (start 102.2 95.1035) (end 102.175 95.0785) (width 0.15) (locked yes) (layer "F.Cu") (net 1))
 (segment (start 102.075 94.3757) (end 101.9 94.2007) (width 0.15) (locked yes) (layer "F.Cu") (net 1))
 (via (at 101.7 92.8) (size 0.6) (drill 0.25) (layers "F.Cu" "B.Cu") (locked yes) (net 1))
 (via (at 101.7 97.8) (size 0.6) (drill 0.25) (layers "F.Cu" "B.Cu") (locked yes) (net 1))
 (segment (start 101.7 92.8) (end 101.7 97.8) (width 0.6) (locked yes) (layer "B.Cu") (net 1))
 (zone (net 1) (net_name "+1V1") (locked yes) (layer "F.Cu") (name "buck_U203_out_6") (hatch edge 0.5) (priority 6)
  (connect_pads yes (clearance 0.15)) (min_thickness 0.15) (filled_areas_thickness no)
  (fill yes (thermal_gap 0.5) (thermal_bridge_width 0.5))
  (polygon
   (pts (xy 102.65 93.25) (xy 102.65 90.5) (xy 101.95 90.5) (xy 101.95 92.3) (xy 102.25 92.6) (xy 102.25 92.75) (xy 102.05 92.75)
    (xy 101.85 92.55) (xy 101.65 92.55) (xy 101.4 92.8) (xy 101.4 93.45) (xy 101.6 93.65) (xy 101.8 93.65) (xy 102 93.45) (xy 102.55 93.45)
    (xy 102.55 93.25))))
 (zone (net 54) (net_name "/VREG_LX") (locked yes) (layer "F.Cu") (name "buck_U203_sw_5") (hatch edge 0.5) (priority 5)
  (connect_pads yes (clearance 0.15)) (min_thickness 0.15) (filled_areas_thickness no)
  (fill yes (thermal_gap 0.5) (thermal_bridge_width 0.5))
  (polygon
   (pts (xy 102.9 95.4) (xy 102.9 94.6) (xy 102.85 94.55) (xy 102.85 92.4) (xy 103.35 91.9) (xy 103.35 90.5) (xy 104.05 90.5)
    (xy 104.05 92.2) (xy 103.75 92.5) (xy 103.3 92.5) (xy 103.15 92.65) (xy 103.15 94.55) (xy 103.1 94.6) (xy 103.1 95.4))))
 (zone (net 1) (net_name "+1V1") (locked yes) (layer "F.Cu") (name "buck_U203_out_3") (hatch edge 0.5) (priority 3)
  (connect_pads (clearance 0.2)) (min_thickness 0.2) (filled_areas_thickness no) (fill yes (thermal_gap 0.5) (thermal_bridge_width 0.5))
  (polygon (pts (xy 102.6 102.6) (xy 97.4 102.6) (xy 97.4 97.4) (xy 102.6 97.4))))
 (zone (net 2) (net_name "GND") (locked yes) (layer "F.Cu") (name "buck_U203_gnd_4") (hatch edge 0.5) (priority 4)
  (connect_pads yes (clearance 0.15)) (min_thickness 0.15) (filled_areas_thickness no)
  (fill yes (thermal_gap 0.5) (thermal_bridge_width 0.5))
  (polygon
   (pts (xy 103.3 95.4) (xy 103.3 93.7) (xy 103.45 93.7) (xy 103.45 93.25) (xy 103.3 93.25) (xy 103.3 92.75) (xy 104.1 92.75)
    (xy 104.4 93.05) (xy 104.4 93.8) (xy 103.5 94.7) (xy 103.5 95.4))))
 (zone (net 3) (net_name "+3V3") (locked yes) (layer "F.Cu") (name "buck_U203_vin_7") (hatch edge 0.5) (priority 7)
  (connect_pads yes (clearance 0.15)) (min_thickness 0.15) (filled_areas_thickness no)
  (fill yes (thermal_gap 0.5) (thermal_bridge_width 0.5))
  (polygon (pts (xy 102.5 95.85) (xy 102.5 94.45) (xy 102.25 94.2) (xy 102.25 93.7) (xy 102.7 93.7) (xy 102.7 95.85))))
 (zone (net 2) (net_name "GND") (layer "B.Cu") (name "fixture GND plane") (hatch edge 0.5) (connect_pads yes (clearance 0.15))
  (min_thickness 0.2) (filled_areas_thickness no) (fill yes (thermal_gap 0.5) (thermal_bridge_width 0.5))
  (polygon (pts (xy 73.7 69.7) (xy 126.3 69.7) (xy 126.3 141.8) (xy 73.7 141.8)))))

